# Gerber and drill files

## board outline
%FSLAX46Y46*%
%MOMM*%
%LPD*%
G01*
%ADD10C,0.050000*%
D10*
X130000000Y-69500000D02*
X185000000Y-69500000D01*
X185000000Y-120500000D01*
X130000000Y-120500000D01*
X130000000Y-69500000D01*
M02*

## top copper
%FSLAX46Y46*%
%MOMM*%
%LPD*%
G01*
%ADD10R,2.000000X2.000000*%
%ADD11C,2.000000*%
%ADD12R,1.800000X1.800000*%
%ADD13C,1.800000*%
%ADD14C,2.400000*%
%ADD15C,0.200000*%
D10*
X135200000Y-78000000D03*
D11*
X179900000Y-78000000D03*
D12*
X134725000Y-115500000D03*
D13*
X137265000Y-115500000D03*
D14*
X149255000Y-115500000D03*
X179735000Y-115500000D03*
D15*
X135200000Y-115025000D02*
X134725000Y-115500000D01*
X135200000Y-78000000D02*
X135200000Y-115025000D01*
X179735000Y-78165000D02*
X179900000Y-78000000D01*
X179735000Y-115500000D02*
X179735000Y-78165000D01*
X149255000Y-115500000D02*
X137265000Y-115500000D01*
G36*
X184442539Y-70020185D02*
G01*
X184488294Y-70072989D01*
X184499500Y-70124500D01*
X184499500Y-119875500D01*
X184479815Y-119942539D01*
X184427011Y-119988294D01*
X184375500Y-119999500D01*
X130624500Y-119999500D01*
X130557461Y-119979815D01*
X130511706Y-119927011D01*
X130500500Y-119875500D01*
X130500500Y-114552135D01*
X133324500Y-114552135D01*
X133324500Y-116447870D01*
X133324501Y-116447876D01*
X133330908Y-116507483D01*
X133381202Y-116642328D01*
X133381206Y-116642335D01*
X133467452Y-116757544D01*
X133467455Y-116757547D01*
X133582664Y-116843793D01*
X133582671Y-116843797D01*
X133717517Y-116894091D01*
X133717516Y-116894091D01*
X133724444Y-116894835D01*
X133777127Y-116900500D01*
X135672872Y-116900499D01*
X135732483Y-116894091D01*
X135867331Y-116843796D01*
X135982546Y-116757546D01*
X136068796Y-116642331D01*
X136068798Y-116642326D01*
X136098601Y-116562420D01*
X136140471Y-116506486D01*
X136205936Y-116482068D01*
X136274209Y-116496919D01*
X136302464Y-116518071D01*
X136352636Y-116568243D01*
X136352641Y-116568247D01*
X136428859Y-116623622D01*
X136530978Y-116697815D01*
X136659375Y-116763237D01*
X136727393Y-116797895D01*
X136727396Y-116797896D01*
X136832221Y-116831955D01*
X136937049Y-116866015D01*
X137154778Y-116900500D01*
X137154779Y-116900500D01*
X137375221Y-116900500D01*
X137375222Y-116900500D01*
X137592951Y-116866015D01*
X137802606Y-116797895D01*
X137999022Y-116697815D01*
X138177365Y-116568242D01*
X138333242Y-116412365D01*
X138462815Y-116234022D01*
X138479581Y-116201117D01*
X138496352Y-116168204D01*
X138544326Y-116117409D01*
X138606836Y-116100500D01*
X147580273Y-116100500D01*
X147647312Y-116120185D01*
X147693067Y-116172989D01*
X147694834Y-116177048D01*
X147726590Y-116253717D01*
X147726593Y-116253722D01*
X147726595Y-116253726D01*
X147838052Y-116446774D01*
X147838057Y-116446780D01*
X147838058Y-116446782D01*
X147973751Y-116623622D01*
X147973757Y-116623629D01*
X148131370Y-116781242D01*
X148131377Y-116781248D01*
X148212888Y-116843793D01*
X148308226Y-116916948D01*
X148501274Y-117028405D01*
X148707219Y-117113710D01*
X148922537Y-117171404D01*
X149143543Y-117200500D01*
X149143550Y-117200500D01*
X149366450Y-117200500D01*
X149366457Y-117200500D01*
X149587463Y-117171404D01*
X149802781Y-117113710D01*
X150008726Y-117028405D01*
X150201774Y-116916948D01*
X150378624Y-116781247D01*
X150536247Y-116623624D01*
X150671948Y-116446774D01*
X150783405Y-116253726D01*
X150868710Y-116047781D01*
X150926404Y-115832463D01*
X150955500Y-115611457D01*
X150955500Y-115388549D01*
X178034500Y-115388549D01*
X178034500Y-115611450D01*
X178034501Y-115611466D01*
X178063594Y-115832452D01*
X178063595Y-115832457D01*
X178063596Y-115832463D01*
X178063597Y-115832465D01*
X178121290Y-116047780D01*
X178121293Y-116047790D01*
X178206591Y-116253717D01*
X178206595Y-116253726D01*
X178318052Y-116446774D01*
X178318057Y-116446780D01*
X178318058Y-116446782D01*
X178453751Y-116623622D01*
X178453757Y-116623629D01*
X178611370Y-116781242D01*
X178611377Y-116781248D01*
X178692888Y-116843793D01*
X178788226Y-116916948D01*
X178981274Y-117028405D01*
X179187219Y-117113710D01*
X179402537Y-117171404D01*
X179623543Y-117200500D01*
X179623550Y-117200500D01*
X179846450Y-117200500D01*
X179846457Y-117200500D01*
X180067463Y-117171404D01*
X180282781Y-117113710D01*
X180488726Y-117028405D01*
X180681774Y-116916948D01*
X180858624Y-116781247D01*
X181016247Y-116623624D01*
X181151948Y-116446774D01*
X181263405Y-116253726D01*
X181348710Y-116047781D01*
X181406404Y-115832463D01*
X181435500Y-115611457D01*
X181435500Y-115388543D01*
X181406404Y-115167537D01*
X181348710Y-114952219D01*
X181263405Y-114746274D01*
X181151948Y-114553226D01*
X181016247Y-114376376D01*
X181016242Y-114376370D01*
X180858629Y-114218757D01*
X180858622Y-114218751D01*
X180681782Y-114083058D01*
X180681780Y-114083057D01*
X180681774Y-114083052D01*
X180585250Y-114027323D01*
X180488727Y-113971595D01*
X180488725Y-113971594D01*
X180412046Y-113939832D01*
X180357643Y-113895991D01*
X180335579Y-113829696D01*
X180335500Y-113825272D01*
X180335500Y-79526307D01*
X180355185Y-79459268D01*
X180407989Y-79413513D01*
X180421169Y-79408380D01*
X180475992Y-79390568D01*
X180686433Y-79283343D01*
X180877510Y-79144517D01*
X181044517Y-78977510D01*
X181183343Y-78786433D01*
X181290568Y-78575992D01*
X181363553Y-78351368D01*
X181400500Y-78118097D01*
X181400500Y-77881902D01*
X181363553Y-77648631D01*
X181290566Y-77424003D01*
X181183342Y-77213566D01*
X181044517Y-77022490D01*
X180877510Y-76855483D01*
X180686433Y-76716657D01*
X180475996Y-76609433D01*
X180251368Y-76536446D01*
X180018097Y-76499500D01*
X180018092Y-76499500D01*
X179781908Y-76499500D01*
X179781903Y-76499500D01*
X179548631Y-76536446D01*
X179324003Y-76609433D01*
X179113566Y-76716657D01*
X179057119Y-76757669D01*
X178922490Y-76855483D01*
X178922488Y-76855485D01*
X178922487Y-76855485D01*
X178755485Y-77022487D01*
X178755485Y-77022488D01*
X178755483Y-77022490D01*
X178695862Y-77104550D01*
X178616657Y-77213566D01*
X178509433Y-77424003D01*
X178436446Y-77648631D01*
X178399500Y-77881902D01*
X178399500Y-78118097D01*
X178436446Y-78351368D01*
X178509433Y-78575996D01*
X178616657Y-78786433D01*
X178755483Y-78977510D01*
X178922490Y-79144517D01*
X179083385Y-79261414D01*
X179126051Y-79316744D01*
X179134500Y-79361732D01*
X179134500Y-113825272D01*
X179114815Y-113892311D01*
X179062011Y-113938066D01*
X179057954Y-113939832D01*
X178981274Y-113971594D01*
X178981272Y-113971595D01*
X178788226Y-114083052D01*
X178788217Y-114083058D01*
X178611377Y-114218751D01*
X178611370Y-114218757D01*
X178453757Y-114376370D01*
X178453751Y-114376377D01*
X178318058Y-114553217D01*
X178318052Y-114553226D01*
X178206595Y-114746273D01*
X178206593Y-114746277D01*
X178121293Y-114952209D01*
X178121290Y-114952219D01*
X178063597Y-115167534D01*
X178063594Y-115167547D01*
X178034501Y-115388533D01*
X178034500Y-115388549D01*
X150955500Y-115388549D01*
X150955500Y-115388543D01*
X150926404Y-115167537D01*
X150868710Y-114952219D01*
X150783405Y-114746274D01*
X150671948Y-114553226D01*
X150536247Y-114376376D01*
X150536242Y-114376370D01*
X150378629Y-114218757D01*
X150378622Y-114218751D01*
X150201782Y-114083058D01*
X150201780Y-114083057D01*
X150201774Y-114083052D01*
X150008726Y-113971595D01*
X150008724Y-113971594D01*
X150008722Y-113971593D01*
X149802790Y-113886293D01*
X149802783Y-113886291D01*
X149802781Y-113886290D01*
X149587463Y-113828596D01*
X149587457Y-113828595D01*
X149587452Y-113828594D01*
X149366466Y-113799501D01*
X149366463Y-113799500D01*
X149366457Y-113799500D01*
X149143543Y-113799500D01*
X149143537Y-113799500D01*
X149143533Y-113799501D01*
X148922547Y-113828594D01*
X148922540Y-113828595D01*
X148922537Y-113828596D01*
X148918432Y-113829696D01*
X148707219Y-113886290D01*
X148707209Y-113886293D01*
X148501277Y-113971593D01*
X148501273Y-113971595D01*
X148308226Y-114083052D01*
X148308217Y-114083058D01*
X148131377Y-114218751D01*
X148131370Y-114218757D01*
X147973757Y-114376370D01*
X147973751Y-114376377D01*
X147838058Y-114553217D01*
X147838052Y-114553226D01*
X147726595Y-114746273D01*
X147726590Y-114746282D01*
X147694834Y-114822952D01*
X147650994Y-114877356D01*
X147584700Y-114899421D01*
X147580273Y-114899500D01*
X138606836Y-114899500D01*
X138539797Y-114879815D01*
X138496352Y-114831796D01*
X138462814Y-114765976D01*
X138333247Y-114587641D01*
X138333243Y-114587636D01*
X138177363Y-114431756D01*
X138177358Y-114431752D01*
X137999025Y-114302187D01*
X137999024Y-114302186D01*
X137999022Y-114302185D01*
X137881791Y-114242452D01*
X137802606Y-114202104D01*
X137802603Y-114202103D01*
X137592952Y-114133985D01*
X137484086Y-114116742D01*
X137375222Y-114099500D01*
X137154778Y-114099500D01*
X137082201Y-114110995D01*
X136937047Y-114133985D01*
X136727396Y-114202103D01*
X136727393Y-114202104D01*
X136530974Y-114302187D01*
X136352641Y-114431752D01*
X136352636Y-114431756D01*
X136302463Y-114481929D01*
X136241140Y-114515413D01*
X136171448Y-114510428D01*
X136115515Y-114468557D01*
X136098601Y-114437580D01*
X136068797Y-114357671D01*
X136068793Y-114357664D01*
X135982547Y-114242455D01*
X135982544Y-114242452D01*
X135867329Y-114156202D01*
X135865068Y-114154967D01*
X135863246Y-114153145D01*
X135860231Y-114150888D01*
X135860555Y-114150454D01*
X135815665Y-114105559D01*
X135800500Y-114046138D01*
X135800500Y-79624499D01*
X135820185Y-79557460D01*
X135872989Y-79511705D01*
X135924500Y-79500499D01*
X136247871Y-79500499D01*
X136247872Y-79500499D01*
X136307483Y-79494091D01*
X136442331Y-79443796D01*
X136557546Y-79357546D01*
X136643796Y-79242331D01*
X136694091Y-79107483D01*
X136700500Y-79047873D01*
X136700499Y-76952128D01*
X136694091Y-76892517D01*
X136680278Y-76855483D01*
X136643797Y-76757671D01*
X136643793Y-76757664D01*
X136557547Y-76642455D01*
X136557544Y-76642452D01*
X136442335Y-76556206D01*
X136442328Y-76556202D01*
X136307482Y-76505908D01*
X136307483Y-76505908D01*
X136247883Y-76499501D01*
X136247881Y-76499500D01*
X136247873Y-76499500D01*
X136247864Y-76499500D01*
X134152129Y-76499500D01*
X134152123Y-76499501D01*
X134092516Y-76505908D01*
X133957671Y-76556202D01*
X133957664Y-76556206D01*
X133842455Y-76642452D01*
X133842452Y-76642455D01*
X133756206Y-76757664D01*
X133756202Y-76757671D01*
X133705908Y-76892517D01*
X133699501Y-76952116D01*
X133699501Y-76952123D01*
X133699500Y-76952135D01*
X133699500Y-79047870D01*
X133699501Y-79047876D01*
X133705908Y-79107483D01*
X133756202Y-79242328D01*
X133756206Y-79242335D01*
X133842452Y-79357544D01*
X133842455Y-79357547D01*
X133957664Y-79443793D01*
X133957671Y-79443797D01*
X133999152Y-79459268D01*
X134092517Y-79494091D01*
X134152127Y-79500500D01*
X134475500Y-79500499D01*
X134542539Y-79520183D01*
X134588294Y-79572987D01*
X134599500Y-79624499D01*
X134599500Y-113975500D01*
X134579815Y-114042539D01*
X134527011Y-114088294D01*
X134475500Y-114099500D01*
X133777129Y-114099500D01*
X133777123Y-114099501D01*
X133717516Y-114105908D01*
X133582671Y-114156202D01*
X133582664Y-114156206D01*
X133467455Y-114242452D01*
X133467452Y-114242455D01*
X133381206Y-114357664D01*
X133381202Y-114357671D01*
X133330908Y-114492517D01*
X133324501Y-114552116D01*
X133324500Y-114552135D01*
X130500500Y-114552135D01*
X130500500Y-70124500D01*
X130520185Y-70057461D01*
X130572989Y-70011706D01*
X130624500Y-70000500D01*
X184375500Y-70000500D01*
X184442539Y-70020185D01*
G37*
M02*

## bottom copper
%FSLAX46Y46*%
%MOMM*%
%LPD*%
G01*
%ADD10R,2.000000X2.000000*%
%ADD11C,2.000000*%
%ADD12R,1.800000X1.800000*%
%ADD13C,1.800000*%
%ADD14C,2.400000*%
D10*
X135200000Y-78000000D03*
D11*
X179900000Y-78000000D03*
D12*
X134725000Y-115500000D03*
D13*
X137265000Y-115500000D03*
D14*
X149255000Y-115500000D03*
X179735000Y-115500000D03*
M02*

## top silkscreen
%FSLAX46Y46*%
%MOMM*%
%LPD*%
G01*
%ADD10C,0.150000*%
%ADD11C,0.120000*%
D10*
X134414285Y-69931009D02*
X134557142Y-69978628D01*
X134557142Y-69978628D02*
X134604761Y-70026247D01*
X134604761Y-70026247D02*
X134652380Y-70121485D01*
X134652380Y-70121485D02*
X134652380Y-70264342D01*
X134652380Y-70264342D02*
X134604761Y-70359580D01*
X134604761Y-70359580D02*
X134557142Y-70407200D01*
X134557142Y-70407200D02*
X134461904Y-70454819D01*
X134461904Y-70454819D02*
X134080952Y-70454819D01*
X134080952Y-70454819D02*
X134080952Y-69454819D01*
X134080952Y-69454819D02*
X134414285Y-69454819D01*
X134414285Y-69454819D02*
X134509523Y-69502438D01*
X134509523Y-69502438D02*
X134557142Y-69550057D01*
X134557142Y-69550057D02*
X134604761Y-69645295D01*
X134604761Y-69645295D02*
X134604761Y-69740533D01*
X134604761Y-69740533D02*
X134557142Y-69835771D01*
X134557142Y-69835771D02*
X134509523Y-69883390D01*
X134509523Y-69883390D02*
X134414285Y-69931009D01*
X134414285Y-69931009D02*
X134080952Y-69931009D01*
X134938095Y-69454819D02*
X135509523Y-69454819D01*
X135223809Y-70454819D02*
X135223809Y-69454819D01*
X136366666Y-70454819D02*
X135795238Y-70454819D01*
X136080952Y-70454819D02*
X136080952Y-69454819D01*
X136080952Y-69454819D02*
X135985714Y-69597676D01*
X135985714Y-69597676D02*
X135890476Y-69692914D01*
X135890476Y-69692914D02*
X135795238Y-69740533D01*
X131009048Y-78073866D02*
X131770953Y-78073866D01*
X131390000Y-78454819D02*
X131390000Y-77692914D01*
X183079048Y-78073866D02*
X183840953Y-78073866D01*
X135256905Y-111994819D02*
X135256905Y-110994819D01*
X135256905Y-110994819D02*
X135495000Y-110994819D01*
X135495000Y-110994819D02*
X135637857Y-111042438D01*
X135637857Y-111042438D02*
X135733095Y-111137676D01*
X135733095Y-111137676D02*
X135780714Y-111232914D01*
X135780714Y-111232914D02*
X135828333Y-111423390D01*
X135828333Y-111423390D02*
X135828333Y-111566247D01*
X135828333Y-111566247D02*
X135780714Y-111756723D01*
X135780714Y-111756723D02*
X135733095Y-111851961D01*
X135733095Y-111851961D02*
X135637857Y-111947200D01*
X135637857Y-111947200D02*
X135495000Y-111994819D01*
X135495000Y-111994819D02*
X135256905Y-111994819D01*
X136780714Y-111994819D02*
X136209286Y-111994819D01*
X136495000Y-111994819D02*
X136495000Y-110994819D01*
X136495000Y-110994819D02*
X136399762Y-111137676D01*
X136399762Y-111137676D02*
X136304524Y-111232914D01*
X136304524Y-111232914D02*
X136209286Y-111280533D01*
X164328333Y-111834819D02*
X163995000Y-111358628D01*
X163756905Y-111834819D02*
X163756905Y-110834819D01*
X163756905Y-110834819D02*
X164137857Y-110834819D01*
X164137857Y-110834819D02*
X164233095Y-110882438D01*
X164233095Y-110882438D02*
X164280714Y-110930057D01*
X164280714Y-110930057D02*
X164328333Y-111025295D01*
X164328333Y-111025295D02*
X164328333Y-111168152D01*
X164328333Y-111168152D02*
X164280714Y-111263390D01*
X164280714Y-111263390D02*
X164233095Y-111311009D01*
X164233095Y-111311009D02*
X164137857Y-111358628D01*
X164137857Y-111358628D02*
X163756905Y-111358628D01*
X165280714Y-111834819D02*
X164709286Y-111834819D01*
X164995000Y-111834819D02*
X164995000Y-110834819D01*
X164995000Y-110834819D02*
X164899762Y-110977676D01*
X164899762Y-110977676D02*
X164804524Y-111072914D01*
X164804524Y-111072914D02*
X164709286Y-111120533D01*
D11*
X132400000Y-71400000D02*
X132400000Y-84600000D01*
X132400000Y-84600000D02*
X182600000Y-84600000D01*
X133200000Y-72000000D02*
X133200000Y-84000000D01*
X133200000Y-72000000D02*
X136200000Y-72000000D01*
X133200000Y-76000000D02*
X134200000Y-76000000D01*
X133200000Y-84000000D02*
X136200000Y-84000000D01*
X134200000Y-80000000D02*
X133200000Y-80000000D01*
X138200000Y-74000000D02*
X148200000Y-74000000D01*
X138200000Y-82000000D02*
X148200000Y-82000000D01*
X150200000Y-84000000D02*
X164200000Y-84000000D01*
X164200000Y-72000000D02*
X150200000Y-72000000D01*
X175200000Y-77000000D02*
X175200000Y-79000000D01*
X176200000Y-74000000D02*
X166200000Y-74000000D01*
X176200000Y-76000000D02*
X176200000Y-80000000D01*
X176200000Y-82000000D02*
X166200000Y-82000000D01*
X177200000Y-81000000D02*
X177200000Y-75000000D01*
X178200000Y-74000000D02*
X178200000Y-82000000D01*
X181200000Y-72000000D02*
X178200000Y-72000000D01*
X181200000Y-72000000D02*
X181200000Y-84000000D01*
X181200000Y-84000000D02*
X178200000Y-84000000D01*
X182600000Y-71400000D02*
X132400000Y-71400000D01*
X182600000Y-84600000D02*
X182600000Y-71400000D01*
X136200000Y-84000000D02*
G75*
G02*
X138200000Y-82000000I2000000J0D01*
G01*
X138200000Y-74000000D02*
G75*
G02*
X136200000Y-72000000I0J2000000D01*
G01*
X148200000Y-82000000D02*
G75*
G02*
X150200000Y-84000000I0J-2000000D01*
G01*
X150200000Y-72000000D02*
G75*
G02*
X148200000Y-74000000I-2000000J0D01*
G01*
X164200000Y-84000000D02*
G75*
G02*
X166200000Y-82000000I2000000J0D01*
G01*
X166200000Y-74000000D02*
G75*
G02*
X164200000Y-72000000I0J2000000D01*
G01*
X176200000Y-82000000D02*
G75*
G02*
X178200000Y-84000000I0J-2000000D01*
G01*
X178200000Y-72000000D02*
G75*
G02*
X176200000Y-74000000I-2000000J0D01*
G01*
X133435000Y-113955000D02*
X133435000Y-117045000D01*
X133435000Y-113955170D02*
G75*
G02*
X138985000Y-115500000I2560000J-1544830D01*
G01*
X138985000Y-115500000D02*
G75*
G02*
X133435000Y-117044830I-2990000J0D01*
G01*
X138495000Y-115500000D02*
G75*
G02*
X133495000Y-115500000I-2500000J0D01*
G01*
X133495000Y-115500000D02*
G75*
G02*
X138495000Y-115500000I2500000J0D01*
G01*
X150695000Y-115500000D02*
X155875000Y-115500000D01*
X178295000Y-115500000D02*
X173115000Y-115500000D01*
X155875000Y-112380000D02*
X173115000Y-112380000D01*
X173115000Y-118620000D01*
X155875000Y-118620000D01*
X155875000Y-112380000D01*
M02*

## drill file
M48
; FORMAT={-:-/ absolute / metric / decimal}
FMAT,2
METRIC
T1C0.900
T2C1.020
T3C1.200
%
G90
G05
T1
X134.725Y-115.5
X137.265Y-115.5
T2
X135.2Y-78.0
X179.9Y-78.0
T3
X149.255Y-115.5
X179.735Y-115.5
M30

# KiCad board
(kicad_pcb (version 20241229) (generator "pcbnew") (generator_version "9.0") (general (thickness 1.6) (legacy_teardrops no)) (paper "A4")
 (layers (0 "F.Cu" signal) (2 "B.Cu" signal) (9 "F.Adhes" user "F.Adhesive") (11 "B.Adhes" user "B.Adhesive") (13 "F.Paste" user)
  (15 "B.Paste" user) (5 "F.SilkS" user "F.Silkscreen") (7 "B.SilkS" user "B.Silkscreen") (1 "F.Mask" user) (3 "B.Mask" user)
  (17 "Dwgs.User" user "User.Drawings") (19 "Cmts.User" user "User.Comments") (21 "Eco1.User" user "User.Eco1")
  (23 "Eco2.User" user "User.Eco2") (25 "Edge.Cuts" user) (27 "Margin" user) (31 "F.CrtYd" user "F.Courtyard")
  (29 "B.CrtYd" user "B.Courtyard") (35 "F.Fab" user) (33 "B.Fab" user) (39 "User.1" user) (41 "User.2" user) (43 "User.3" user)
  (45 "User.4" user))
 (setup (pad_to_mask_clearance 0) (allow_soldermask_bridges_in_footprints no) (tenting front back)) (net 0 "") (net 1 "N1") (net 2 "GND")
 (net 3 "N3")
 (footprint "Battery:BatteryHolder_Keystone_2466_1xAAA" (layer "F.Cu") (at 135.2 78)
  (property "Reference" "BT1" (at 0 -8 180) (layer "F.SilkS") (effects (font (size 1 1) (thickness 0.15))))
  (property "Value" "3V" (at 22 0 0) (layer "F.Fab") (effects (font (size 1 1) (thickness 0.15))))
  (fp_line (start -2.8 -6.6) (end -2.8 6.6) (stroke (width 0.12) (type solid)) (layer "F.SilkS"))
  (fp_line (start -2.8 6.6) (end 47.4 6.6) (stroke (width 0.12) (type solid)) (layer "F.SilkS"))
  (fp_line (start -2 -6) (end -2 6) (stroke (width 0.12) (type solid)) (layer "F.SilkS"))
  (fp_line (start -2 -6) (end 1 -6) (stroke (width 0.12) (type solid)) (layer "F.SilkS"))
  (fp_line (start -2 -2) (end -1 -2) (stroke (width 0.12) (type solid)) (layer "F.SilkS"))
  (fp_line (start -2 6) (end 1 6) (stroke (width 0.12) (type solid)) (layer "F.SilkS"))
  (fp_line (start -1 2) (end -2 2) (stroke (width 0.12) (type solid)) (layer "F.SilkS"))
  (fp_line (start 3 -4) (end 13 -4) (stroke (width 0.12) (type solid)) (layer "F.SilkS"))
  (fp_line (start 3 4) (end 13 4) (stroke (width 0.12) (type solid)) (layer "F.SilkS"))
  (fp_line (start 15 6) (end 29 6) (stroke (width 0.12) (type solid)) (layer "F.SilkS"))
  (fp_line (start 29 -6) (end 15 -6) (stroke (width 0.12) (type solid)) (layer "F.SilkS"))
  (fp_line (start 40 -1) (end 40 1) (stroke (width 0.12) (type solid)) (layer "F.SilkS"))
  (fp_line (start 41 -4) (end 31 -4) (stroke (width 0.12) (type solid)) (layer "F.SilkS"))
  (fp_line (start 41 -2) (end 41 2) (stroke (width 0.12) (type solid)) (layer "F.SilkS"))
  (fp_line (start 41 4) (end 31 4) (stroke (width 0.12) (type solid)) (layer "F.SilkS"))
  (fp_line (start 42 3) (end 42 -3) (stroke (width 0.12) (type solid)) (layer "F.SilkS"))
  (fp_line (start 43 -4) (end 43 4) (stroke (width 0.12) (type solid)) (layer "F.SilkS"))
  (fp_line (start 46 -6) (end 43 -6) (stroke (width 0.12) (type solid)) (layer "F.SilkS"))
  (fp_line (start 46 -6) (end 46 6) (stroke (width 0.12) (type solid)) (layer "F.SilkS"))
  (fp_line (start 46 6) (end 43 6) (stroke (width 0.12) (type solid)) (layer "F.SilkS"))
  (fp_line (start 47.4 -6.6) (end -2.8 -6.6) (stroke (width 0.12) (type solid)) (layer "F.SilkS"))
  (fp_line (start 47.4 6.6) (end 47.4 -6.6) (stroke (width 0.12) (type solid)) (layer "F.SilkS"))
  (fp_arc (start 1 6) (mid 1.585786 4.585786) (end 3 4) (stroke (width 0.12) (type solid)) (layer "F.SilkS"))
  (fp_arc (start 3 -4) (mid 1.585786 -4.585786) (end 1 -6) (stroke (width 0.12) (type solid)) (layer "F.SilkS"))
  (fp_arc (start 13 4) (mid 14.414214 4.585786) (end 15 6) (stroke (width 0.12) (type solid)) (layer "F.SilkS"))
  (fp_arc (start 15 -6) (mid 14.414214 -4.585786) (end 13 -4) (stroke (width 0.12) (type solid)) (layer "F.SilkS"))
  (fp_arc (start 29 6) (mid 29.585786 4.585786) (end 31 4) (stroke (width 0.12) (type solid)) (layer "F.SilkS"))
  (fp_arc (start 31 -4) (mid 29.585786 -4.585786) (end 29 -6) (stroke (width 0.12) (type solid)) (layer "F.SilkS"))
  (fp_arc (start 41 4) (mid 42.414214 4.585786) (end 43 6) (stroke (width 0.12) (type solid)) (layer "F.SilkS"))
  (fp_arc (start 43 -6) (mid 42.414214 -4.585786) (end 41 -4) (stroke (width 0.12) (type solid)) (layer "F.SilkS"))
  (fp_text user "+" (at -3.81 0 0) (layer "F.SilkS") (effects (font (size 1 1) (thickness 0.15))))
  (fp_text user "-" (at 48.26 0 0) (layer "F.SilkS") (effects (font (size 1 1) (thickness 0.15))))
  (pad "1" thru_hole rect (at 0 0) (size 2 2) (drill 1.02) (layers "*.Cu" "*.Mask") (remove_unused_layers no) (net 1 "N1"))
  (pad "2" thru_hole circle (at 44.7 0) (size 2 2) (drill 1.02) (layers "*.Cu" "*.Mask") (remove_unused_layers no) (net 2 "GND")))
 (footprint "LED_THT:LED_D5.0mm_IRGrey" (layer "F.Cu") (at 134.725 115.5)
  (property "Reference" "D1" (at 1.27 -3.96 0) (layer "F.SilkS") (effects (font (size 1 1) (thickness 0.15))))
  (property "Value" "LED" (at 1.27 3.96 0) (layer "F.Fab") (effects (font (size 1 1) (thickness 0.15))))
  (fp_line (start -1.29 -1.545) (end -1.29 1.545) (stroke (width 0.12) (type solid)) (layer "F.SilkS"))
  (fp_arc (start -1.29 -1.54483) (mid 2.071779 -2.880495) (end 4.26 0) (stroke (width 0.12) (type solid)) (layer "F.SilkS"))
  (fp_arc (start 4.26 0) (mid 2.071779 2.880495) (end -1.29 1.54483) (stroke (width 0.12) (type solid)) (layer "F.SilkS"))
  (fp_circle (center 1.27 0) (end 3.77 0) (stroke (width 0.12) (type solid)) (fill no) (layer "F.SilkS"))
  (pad "1" thru_hole rect (at 0 0) (size 1.8 1.8) (drill 0.9) (layers "*.Cu" "*.Mask") (remove_unused_layers no) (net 1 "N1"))
  (pad "2" thru_hole circle (at 2.54 0) (size 1.8 1.8) (drill 0.9) (layers "*.Cu" "*.Mask") (remove_unused_layers no) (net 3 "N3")))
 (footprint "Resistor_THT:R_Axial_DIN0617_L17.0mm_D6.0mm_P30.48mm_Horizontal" (layer "F.Cu") (at 149.255 115.5)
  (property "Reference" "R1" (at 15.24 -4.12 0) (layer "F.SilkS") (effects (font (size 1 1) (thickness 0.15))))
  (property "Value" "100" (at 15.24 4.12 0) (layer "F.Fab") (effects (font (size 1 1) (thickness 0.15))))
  (fp_line (start 1.44 0) (end 6.62 0) (stroke (width 0.12) (type solid)) (layer "F.SilkS"))
  (fp_line (start 29.04 0) (end 23.86 0) (stroke (width 0.12) (type solid)) (layer "F.SilkS"))
  (fp_rect (start 6.62 -3.12) (end 23.86 3.12) (stroke (width 0.12) (type solid)) (fill no) (layer "F.SilkS"))
  (pad "1" thru_hole circle (at 0 0) (size 2.4 2.4) (drill 1.2) (layers "*.Cu" "*.Mask") (remove_unused_layers no) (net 3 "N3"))
  (pad "2" thru_hole circle (at 30.48 0) (size 2.4 2.4) (drill 1.2) (layers "*.Cu" "*.Mask") (remove_unused_layers no) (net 2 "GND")))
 (gr_rect (start 130 69.5) (end 185 120.5) (stroke (width 0.05) (type default)) (fill no) (layer "Edge.Cuts"))
 (segment (start 135.2 115.025) (end 134.725 115.5) (width 0.2) (layer "F.Cu") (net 1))
 (segment (start 135.2 78) (end 135.2 115.025) (width 0.2) (layer "F.Cu") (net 1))
 (segment (start 179.735 78.165) (end 179.9 78) (width 0.2) (layer "F.Cu") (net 2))
 (segment (start 179.735 115.5) (end 179.735 78.165) (width 0.2) (layer "F.Cu") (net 2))
 (segment (start 149.255 115.5) (end 137.265 115.5) (width 0.2) (layer "F.Cu") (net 3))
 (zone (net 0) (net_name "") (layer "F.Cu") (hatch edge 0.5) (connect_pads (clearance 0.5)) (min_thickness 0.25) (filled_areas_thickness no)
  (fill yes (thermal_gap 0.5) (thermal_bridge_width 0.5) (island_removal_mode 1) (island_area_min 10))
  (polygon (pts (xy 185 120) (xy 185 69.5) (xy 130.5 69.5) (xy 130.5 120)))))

